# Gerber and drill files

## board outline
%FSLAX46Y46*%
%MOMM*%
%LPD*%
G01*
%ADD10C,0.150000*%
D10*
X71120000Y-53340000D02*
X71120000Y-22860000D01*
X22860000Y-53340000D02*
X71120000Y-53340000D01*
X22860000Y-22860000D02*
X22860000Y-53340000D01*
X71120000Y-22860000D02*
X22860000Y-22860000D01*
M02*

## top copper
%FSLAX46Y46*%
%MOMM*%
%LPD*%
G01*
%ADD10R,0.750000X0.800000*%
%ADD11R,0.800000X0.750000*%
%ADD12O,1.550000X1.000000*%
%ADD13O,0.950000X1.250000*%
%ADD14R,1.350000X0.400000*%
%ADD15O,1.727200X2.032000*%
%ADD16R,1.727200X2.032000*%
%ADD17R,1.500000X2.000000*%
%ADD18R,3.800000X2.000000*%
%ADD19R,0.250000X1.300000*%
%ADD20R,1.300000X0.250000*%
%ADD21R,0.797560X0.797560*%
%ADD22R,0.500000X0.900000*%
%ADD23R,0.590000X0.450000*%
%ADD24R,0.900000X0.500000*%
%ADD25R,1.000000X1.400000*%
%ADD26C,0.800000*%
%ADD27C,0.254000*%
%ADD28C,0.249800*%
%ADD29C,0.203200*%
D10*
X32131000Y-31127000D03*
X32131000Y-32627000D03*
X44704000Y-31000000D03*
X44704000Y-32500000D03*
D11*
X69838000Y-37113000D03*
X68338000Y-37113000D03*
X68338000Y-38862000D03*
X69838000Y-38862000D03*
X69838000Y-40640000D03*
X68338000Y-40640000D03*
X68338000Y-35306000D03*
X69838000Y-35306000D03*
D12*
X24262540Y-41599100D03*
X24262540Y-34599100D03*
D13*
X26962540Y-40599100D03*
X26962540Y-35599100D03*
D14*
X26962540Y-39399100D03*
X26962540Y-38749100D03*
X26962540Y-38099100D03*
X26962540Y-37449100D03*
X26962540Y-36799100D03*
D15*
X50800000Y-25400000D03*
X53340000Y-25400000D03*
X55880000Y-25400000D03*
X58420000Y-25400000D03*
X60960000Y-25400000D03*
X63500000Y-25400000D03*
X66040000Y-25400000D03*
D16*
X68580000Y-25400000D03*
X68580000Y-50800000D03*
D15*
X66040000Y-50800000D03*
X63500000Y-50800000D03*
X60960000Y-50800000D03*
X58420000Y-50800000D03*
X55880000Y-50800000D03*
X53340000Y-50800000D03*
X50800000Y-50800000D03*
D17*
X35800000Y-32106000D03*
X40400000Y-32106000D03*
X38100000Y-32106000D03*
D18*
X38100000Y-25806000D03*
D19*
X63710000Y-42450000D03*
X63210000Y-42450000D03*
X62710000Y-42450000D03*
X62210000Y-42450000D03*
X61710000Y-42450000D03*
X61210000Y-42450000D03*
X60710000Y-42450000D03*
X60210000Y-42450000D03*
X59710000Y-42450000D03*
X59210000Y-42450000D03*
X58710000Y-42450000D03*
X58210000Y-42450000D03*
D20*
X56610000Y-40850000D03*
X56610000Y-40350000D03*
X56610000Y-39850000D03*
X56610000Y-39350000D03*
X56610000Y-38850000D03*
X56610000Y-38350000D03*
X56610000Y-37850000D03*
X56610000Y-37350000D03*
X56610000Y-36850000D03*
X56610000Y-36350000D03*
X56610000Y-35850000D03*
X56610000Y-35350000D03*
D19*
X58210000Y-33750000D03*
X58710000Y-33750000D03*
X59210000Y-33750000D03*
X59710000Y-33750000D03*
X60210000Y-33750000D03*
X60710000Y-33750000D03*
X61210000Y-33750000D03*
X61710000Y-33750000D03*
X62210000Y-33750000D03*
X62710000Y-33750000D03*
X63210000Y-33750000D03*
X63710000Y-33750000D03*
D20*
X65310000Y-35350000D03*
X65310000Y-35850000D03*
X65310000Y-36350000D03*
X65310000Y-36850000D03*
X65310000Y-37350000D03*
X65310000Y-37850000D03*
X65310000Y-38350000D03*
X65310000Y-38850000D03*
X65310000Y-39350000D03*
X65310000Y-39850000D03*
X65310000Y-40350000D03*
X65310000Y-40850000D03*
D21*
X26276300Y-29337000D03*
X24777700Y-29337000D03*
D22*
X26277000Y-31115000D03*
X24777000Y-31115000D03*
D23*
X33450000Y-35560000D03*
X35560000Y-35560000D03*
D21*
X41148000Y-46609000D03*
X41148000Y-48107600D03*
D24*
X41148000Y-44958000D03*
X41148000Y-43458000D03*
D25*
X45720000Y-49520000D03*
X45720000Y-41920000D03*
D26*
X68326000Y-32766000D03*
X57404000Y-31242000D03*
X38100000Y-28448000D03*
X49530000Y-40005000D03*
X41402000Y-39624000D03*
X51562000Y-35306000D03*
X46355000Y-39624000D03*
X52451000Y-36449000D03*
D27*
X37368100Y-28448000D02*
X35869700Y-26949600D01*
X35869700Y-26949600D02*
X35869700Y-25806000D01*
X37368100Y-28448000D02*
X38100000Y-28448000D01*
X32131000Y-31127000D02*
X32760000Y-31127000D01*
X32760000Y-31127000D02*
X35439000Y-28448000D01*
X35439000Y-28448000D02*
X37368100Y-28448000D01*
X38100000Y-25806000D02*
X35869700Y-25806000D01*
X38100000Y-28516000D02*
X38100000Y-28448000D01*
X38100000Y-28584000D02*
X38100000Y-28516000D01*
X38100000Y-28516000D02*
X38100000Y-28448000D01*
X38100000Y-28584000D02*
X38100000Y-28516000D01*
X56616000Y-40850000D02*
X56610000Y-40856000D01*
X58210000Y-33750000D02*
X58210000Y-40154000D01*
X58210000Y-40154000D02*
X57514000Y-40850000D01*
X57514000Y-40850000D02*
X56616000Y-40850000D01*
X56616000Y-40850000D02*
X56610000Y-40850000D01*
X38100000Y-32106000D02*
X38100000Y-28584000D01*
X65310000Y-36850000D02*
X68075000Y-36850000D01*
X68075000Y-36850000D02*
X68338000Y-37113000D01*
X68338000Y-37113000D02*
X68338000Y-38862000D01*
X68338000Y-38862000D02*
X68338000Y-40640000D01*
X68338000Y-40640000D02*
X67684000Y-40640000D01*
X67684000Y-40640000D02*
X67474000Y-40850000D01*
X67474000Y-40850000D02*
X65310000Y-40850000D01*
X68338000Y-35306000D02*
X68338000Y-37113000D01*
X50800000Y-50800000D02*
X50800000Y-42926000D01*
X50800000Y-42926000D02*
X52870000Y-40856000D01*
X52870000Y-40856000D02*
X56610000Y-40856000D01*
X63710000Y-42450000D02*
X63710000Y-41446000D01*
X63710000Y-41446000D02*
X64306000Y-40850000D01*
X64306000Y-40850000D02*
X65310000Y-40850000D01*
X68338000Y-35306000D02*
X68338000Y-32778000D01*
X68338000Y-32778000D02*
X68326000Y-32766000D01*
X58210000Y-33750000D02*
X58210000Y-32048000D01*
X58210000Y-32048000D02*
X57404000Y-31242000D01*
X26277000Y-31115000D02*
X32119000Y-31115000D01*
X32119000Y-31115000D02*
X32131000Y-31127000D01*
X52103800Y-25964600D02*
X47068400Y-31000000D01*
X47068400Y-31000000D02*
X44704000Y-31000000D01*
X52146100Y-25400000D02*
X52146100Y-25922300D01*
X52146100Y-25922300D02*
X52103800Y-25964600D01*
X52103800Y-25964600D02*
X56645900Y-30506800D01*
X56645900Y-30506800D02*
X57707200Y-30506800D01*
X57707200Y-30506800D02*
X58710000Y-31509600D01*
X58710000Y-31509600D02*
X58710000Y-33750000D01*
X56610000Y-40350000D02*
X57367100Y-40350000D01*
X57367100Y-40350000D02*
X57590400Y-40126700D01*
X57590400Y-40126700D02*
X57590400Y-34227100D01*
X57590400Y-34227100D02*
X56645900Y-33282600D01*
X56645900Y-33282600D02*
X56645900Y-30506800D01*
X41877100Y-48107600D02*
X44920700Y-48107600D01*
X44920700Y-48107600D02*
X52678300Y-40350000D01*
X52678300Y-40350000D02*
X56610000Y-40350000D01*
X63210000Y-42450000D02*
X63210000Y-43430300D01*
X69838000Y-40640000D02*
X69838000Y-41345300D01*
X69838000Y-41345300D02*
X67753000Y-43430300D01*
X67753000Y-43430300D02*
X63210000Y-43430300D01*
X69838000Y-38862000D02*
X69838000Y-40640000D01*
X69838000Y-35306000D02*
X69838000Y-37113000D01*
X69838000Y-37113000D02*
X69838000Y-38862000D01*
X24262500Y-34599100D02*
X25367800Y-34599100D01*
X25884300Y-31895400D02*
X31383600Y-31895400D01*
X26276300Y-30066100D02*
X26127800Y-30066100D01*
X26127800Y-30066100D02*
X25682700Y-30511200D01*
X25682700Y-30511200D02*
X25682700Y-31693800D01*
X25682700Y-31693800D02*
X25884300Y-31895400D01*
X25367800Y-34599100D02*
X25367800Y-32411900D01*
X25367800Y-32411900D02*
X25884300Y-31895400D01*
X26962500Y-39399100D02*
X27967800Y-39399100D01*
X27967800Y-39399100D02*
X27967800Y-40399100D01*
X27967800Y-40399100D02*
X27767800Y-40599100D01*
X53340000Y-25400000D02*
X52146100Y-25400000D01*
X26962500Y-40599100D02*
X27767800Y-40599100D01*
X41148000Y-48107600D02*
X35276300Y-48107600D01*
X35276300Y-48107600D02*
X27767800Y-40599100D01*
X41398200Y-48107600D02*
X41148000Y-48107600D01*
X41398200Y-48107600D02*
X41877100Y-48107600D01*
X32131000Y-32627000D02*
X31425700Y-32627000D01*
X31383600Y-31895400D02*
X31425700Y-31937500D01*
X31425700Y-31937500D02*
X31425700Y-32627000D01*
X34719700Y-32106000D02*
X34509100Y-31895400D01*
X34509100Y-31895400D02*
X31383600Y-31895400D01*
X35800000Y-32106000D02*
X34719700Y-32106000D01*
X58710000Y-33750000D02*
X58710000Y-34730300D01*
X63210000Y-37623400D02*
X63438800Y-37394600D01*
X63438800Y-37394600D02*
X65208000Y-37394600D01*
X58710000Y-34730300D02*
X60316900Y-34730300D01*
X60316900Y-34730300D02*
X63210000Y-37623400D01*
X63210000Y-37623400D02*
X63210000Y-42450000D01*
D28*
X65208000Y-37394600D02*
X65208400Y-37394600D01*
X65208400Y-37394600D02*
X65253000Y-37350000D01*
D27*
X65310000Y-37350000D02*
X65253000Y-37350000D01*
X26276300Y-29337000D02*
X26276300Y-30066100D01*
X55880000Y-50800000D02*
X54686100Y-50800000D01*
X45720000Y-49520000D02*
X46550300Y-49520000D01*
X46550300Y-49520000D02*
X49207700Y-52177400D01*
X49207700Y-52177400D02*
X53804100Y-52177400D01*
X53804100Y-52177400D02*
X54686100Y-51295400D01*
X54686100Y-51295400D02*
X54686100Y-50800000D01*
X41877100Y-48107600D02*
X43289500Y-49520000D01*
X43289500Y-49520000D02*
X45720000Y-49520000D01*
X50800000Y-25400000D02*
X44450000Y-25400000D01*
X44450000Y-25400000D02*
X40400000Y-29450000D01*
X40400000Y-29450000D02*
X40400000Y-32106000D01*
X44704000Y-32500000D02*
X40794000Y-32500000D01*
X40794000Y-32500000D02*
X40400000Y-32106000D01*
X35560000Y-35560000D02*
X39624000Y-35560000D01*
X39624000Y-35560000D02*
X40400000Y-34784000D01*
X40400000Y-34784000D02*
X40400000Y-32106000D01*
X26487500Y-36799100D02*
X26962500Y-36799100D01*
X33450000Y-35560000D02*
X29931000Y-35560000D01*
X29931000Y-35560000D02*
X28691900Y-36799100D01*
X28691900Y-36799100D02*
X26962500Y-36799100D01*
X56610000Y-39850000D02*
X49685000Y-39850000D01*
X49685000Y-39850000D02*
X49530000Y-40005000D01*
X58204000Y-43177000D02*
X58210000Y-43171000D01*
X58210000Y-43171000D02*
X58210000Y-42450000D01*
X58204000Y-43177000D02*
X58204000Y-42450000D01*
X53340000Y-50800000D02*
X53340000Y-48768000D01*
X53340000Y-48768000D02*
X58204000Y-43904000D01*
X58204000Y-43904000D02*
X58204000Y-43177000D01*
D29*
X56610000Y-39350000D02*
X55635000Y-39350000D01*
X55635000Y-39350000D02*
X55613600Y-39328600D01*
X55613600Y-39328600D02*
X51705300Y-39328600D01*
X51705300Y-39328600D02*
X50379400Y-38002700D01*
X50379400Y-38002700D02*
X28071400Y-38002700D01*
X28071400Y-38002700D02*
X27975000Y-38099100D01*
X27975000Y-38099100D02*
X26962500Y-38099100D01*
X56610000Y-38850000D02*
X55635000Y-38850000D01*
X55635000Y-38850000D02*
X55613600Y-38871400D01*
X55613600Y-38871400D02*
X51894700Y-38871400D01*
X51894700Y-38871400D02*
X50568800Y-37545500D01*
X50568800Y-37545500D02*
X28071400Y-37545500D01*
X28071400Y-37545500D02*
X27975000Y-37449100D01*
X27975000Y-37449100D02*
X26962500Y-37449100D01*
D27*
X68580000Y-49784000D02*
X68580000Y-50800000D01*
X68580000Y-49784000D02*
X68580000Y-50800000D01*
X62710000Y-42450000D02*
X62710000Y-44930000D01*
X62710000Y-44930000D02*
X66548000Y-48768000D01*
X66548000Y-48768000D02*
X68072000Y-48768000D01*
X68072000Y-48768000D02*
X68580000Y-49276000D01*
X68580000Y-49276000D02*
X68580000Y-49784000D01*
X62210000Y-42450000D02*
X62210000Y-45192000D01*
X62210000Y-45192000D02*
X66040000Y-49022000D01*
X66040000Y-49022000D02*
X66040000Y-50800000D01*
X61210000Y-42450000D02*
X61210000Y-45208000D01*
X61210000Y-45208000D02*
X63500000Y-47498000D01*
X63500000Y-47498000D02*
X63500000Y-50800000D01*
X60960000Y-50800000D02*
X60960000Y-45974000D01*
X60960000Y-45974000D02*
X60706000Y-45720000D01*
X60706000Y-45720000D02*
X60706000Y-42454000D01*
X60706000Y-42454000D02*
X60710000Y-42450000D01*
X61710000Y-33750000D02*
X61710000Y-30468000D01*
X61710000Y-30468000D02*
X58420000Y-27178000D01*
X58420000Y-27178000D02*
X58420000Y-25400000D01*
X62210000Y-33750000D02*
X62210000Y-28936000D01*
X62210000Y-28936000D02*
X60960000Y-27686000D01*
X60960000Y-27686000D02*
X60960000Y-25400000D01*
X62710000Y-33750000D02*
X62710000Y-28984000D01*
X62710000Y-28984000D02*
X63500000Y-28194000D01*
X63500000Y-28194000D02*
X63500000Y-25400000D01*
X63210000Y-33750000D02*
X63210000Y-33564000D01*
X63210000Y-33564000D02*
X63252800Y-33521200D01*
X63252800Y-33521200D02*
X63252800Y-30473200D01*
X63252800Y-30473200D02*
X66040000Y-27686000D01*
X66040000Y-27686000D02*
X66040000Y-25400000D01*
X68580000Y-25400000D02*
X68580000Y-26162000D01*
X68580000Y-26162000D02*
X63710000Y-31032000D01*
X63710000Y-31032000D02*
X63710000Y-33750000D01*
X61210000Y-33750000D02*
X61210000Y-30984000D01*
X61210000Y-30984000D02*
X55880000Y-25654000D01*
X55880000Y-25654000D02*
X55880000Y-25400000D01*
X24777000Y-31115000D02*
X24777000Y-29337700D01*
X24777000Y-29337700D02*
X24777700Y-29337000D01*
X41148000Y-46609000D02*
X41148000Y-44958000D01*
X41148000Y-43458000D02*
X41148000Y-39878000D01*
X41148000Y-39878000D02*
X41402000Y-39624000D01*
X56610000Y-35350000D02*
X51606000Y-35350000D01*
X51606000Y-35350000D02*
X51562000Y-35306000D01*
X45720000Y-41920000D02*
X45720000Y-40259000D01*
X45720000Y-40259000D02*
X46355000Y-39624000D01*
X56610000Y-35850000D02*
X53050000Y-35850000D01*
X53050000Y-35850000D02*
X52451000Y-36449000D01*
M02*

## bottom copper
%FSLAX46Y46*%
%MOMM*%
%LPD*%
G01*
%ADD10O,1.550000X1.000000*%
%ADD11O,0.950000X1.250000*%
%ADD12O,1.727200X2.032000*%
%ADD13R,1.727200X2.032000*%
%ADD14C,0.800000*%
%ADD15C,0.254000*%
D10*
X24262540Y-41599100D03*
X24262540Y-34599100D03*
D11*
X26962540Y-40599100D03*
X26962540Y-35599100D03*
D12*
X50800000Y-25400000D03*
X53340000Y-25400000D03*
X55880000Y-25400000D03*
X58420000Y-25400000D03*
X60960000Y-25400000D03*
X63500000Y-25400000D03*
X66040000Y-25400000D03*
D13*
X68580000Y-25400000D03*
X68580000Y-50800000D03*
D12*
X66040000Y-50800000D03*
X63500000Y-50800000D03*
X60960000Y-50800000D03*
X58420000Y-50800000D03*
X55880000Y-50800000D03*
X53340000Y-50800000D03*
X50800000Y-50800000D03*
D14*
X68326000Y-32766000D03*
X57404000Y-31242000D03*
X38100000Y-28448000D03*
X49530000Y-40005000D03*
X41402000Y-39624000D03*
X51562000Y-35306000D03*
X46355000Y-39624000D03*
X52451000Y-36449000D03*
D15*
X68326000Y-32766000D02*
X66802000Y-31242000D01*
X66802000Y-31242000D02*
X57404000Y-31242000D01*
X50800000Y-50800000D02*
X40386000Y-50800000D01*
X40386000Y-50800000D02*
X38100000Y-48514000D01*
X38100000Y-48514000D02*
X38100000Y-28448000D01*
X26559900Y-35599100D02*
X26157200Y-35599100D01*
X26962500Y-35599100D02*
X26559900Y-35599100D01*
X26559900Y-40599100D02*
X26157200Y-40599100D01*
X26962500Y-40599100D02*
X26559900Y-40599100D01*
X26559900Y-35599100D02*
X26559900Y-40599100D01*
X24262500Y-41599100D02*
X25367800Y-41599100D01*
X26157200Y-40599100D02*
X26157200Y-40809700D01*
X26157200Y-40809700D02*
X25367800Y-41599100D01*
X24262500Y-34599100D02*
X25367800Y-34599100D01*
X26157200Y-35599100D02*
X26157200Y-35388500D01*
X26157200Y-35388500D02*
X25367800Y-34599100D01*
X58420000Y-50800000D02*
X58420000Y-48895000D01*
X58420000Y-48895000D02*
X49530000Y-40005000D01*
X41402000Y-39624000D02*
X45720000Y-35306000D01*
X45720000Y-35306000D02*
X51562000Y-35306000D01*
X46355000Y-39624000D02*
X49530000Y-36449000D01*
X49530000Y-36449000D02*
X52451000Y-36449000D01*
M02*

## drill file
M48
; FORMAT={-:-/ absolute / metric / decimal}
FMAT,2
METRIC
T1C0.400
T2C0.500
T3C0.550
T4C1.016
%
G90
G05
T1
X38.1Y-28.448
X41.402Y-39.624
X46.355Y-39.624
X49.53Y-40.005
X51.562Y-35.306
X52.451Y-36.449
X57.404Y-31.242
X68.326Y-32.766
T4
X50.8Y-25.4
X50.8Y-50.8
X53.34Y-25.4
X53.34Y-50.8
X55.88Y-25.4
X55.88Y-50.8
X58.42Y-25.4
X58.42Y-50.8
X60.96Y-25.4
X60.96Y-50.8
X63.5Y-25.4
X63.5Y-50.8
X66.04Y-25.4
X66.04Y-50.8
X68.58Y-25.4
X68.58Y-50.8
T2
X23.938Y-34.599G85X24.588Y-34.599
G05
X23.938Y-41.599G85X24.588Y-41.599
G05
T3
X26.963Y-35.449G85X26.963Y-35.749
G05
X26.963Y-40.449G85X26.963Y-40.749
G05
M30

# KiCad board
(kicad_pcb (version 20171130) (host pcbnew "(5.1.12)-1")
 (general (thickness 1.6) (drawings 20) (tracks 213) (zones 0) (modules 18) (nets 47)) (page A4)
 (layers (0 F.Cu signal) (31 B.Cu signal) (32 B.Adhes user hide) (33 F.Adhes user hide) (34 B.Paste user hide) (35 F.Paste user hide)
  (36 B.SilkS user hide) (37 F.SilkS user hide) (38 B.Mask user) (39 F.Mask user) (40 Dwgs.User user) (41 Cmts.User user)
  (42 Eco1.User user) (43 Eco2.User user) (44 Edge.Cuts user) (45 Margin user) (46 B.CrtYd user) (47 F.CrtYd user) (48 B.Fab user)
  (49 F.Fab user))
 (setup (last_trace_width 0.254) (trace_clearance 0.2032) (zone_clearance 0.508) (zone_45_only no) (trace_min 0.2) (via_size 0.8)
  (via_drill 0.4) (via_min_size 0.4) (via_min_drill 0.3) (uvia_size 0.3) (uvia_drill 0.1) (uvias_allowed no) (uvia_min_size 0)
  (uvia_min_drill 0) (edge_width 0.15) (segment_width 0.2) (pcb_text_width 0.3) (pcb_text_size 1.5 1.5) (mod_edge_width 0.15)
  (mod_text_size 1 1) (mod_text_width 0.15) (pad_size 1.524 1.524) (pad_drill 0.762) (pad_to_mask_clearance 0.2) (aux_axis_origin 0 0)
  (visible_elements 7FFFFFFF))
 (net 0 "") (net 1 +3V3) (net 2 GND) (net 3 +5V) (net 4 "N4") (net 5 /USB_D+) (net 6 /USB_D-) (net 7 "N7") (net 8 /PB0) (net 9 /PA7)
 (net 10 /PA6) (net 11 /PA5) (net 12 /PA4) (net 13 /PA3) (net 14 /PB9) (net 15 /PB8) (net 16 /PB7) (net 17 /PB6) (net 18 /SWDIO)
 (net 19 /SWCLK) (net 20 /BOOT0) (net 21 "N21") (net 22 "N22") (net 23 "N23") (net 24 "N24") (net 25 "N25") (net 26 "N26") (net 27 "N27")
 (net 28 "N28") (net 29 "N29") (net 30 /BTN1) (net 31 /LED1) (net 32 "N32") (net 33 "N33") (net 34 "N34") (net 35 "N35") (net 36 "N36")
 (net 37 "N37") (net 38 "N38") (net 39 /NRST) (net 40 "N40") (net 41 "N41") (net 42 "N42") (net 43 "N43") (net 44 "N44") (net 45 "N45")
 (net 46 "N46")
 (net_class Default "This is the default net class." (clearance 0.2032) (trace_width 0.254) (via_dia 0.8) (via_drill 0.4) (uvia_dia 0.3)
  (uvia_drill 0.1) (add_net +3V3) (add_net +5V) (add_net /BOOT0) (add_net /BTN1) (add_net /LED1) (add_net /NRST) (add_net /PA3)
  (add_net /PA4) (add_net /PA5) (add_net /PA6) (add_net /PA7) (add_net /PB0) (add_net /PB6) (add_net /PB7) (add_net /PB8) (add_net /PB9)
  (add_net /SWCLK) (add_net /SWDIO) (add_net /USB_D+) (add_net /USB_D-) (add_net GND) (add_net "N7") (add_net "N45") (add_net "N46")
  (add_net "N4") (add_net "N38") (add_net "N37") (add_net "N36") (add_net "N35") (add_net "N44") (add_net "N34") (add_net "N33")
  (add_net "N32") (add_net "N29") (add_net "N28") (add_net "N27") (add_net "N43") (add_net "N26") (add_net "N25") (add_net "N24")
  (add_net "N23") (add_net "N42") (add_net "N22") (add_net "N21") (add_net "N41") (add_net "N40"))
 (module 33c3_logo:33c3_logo (layer F.Cu) (at 31.75 46.101)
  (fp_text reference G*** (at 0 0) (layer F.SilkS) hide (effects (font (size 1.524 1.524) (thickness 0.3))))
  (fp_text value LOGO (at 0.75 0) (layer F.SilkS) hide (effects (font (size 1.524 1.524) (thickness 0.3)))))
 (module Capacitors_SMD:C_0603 (layer F.Cu) (at 32.131 31.877 270)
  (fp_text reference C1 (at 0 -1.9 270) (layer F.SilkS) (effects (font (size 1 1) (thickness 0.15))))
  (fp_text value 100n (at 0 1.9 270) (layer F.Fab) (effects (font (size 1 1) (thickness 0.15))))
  (pad 1 smd rect (at -0.75 0 270) (size 0.8 0.75) (layers F.Cu F.Paste F.Mask) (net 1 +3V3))
  (pad 2 smd rect (at 0.75 0 270) (size 0.8 0.75) (layers F.Cu F.Paste F.Mask) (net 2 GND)))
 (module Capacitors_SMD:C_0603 (layer F.Cu) (at 44.704 31.75 90)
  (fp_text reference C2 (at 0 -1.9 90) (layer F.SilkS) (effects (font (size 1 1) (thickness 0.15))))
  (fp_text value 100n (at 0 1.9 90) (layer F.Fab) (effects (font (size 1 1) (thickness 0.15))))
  (pad 2 smd rect (at 0.75 0 90) (size 0.8 0.75) (layers F.Cu F.Paste F.Mask) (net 2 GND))
  (pad 1 smd rect (at -0.75 0 90) (size 0.8 0.75) (layers F.Cu F.Paste F.Mask) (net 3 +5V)))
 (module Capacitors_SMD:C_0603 (layer F.Cu) (at 69.088 37.113)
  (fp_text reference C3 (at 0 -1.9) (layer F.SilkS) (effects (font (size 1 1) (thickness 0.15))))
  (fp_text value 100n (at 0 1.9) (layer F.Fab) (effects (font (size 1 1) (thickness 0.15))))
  (pad 2 smd rect (at 0.75 0) (size 0.8 0.75) (layers F.Cu F.Paste F.Mask) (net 2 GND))
  (pad 1 smd rect (at -0.75 0) (size 0.8 0.75) (layers F.Cu F.Paste F.Mask) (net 1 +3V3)))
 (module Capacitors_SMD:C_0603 (layer F.Cu) (at 69.088 38.862)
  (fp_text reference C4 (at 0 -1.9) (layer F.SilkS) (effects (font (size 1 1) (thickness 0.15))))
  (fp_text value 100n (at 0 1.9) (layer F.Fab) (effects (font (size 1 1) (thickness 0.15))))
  (pad 1 smd rect (at -0.75 0) (size 0.8 0.75) (layers F.Cu F.Paste F.Mask) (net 1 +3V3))
  (pad 2 smd rect (at 0.75 0) (size 0.8 0.75) (layers F.Cu F.Paste F.Mask) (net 2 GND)))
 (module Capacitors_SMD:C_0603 (layer F.Cu) (at 69.088 40.64)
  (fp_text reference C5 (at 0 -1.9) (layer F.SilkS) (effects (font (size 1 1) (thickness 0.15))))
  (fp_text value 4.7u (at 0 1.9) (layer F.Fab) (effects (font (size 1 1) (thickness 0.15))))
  (pad 2 smd rect (at 0.75 0) (size 0.8 0.75) (layers F.Cu F.Paste F.Mask) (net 2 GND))
  (pad 1 smd rect (at -0.75 0) (size 0.8 0.75) (layers F.Cu F.Paste F.Mask) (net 1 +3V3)))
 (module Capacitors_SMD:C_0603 (layer F.Cu) (at 69.088 35.306)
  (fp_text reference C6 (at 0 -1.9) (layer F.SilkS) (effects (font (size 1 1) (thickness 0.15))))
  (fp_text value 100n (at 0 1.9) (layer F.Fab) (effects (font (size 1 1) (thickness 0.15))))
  (pad 1 smd rect (at -0.75 0) (size 0.8 0.75) (layers F.Cu F.Paste F.Mask) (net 1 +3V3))
  (pad 2 smd rect (at 0.75 0) (size 0.8 0.75) (layers F.Cu F.Paste F.Mask) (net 2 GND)))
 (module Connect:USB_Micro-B (layer F.Cu) (at 25.4 38.1 270)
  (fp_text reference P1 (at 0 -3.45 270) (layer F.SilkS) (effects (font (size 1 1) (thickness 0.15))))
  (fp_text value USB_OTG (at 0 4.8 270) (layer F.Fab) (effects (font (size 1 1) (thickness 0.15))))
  (pad 6 thru_hole oval (at 3.4991 1.13746) (size 1.55 1) (drill oval 1.15 0.5) (layers *.Cu *.Mask) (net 2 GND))
  (pad 6 thru_hole oval (at -3.5009 1.13746) (size 1.55 1) (drill oval 1.15 0.5) (layers *.Cu *.Mask) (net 2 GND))
  (pad 6 thru_hole oval (at 2.4991 -1.56254) (size 0.95 1.25) (drill oval 0.55 0.85) (layers *.Cu *.Mask) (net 2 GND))
  (pad 6 thru_hole oval (at -2.5009 -1.56254) (size 0.95 1.25) (drill oval 0.55 0.85) (layers *.Cu *.Mask) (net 2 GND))
  (pad 5 smd rect (at 1.2991 -1.56254) (size 1.35 0.4) (layers F.Cu F.Paste F.Mask) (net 2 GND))
  (pad 4 smd rect (at 0.6491 -1.56254) (size 1.35 0.4) (layers F.Cu F.Paste F.Mask) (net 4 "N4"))
  (pad 3 smd rect (at -0.0009 -1.56254) (size 1.35 0.4) (layers F.Cu F.Paste F.Mask) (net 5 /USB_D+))
  (pad 2 smd rect (at -0.6509 -1.56254) (size 1.35 0.4) (layers F.Cu F.Paste F.Mask) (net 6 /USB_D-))
  (pad 1 smd rect (at -1.3009 -1.56254) (size 1.35 0.4) (layers F.Cu F.Paste F.Mask) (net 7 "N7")))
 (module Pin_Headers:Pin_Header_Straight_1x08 (layer F.Cu) (at 68.58 25.4 270)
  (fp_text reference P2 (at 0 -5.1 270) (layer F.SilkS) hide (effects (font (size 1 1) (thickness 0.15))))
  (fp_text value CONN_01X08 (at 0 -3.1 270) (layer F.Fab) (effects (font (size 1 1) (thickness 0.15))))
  (pad 8 thru_hole oval (at 0 17.78 270) (size 2.032 1.7272) (drill 1.016) (layers *.Cu *.Mask) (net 3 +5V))
  (pad 7 thru_hole oval (at 0 15.24 270) (size 2.032 1.7272) (drill 1.016) (layers *.Cu *.Mask) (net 2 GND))
  (pad 6 thru_hole oval (at 0 12.7 270) (size 2.032 1.7272) (drill 1.016) (layers *.Cu *.Mask) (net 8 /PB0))
  (pad 5 thru_hole oval (at 0 10.16 270) (size 2.032 1.7272) (drill 1.016) (layers *.Cu *.Mask) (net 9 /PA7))
  (pad 4 thru_hole oval (at 0 7.62 270) (size 2.032 1.7272) (drill 1.016) (layers *.Cu *.Mask) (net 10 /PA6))
  (pad 3 thru_hole oval (at 0 5.08 270) (size 2.032 1.7272) (drill 1.016) (layers *.Cu *.Mask) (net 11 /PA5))
  (pad 2 thru_hole oval (at 0 2.54 270) (size 2.032 1.7272) (drill 1.016) (layers *.Cu *.Mask) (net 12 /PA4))
  (pad 1 thru_hole rect (at 0 0 270) (size 2.032 1.7272) (drill 1.016) (layers *.Cu *.Mask) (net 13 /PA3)))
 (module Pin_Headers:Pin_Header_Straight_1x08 (layer F.Cu) (at 68.58 50.8 270)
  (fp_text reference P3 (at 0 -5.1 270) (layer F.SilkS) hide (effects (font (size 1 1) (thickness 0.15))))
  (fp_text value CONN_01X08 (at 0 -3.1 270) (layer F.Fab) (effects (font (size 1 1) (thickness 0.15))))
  (pad 1 thru_hole rect (at 0 0 270) (size 2.032 1.7272) (drill 1.016) (layers *.Cu *.Mask) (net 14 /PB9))
  (pad 2 thru_hole oval (at 0 2.54 270) (size 2.032 1.7272) (drill 1.016) (layers *.Cu *.Mask) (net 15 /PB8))
  (pad 3 thru_hole oval (at 0 5.08 270) (size 2.032 1.7272) (drill 1.016) (layers *.Cu *.Mask) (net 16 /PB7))
  (pad 4 thru_hole oval (at 0 7.62 270) (size 2.032 1.7272) (drill 1.016) (layers *.Cu *.Mask) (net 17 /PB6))
  (pad 5 thru_hole oval (at 0 10.16 270) (size 2.032 1.7272) (drill 1.016) (layers *.Cu *.Mask) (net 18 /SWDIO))
  (pad 6 thru_hole oval (at 0 12.7 270) (size 2.032 1.7272) (drill 1.016) (layers *.Cu *.Mask) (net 2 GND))
  (pad 7 thru_hole oval (at 0 15.24 270) (size 2.032 1.7272) (drill 1.016) (layers *.Cu *.Mask) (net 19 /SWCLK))
  (pad 8 thru_hole oval (at 0 17.78 270) (size 2.032 1.7272) (drill 1.016) (layers *.Cu *.Mask) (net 1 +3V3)))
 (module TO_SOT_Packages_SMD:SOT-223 (layer F.Cu) (at 38.1 28.956 90)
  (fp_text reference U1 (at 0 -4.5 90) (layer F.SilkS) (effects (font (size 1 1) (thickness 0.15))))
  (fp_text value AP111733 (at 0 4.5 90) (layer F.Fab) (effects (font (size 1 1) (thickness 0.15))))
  (pad 1 smd rect (at -3.15 -2.3 90) (size 2 1.5) (layers F.Cu F.Paste F.Mask) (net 2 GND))
  (pad 3 smd rect (at -3.15 2.3 90) (size 2 1.5) (layers F.Cu F.Paste F.Mask) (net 3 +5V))
  (pad 2 smd rect (at -3.15 0 90) (size 2 1.5) (layers F.Cu F.Paste F.Mask) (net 1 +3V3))
  (pad 4 smd rect (at 3.15 0 90) (size 2 3.8) (layers F.Cu F.Paste F.Mask) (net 1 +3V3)))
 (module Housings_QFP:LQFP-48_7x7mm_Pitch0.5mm (layer F.Cu) (at 60.96 38.1 180)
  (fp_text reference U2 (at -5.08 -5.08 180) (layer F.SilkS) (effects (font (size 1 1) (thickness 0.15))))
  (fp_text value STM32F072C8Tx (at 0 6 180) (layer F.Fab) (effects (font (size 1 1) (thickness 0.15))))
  (pad 48 smd rect (at -2.75 -4.35 270) (size 1.3 0.25) (layers F.Cu F.Paste F.Mask) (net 1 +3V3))
  (pad 47 smd rect (at -2.25 -4.35 270) (size 1.3 0.25) (layers F.Cu F.Paste F.Mask) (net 2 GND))
  (pad 46 smd rect (at -1.75 -4.35 270) (size 1.3 0.25) (layers F.Cu F.Paste F.Mask) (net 14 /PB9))
  (pad 45 smd rect (at -1.25 -4.35 270) (size 1.3 0.25) (layers F.Cu F.Paste F.Mask) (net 15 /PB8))
  (pad 44 smd rect (at -0.75 -4.35 270) (size 1.3 0.25) (layers F.Cu F.Paste F.Mask) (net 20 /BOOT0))
  (pad 43 smd rect (at -0.25 -4.35 270) (size 1.3 0.25) (layers F.Cu F.Paste F.Mask) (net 16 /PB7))
  (pad 42 smd rect (at 0.25 -4.35 270) (size 1.3 0.25) (layers F.Cu F.Paste F.Mask) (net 17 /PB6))
  (pad 41 smd rect (at 0.75 -4.35 270) (size 1.3 0.25) (layers F.Cu F.Paste F.Mask) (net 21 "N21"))
  (pad 40 smd rect (at 1.25 -4.35 270) (size 1.3 0.25) (layers F.Cu F.Paste F.Mask) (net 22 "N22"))
  (pad 39 smd rect (at 1.75 -4.35 270) (size 1.3 0.25) (layers F.Cu F.Paste F.Mask) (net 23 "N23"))
  (pad 38 smd rect (at 2.25 -4.35 270) (size 1.3 0.25) (layers F.Cu F.Paste F.Mask) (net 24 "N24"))
  (pad 37 smd rect (at 2.75 -4.35 270) (size 1.3 0.25) (layers F.Cu F.Paste F.Mask) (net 19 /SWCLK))
  (pad 36 smd rect (at 4.35 -2.75 180) (size 1.3 0.25) (layers F.Cu F.Paste F.Mask) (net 1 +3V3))
  (pad 35 smd rect (at 4.35 -2.25 180) (size 1.3 0.25) (layers F.Cu F.Paste F.Mask) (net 2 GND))
  (pad 34 smd rect (at 4.35 -1.75 180) (size 1.3 0.25) (layers F.Cu F.Paste F.Mask) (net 18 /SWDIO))
  (pad 33 smd rect (at 4.35 -1.25 180) (size 1.3 0.25) (layers F.Cu F.Paste F.Mask) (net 5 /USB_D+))
  (pad 32 smd rect (at 4.35 -0.75 180) (size 1.3 0.25) (layers F.Cu F.Paste F.Mask) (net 6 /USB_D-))
  (pad 31 smd rect (at 4.35 -0.25 180) (size 1.3 0.25) (layers F.Cu F.Paste F.Mask) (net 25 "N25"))
  (pad 30 smd rect (at 4.35 0.25 180) (size 1.3 0.25) (layers F.Cu F.Paste F.Mask) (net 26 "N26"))
  (pad 29 smd rect (at 4.35 0.75 180) (size 1.3 0.25) (layers F.Cu F.Paste F.Mask) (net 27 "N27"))
  (pad 28 smd rect (at 4.35 1.25 180) (size 1.3 0.25) (layers F.Cu F.Paste F.Mask) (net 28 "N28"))
  (pad 27 smd rect (at 4.35 1.75 180) (size 1.3 0.25) (layers F.Cu F.Paste F.Mask) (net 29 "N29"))
  (pad 26 smd rect (at 4.35 2.25 180) (size 1.3 0.25) (layers F.Cu F.Paste F.Mask) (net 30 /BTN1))
  (pad 25 smd rect (at 4.35 2.75 180) (size 1.3 0.25) (layers F.Cu F.Paste F.Mask) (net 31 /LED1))
  (pad 24 smd rect (at 2.75 4.35 270) (size 1.3 0.25) (layers F.Cu F.Paste F.Mask) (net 1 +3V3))
  (pad 23 smd rect (at 2.25 4.35 270) (size 1.3 0.25) (layers F.Cu F.Paste F.Mask) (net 2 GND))
  (pad 22 smd rect (at 1.75 4.35 270) (size 1.3 0.25) (layers F.Cu F.Paste F.Mask) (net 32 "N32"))
  (pad 21 smd rect (at 1.25 4.35 270) (size 1.3 0.25) (layers F.Cu F.Paste F.Mask) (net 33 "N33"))
  (pad 20 smd rect (at 0.75 4.35 270) (size 1.3 0.25) (layers F.Cu F.Paste F.Mask) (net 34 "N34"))
  (pad 19 smd rect (at 0.25 4.35 270) (size 1.3 0.25) (layers F.Cu F.Paste F.Mask) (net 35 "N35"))
  (pad 18 smd rect (at -0.25 4.35 270) (size 1.3 0.25) (layers F.Cu F.Paste F.Mask) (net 8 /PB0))
  (pad 17 smd rect (at -0.75 4.35 270) (size 1.3 0.25) (layers F.Cu F.Paste F.Mask) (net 9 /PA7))
  (pad 16 smd rect (at -1.25 4.35 270) (size 1.3 0.25) (layers F.Cu F.Paste F.Mask) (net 10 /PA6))
  (pad 15 smd rect (at -1.75 4.35 270) (size 1.3 0.25) (layers F.Cu F.Paste F.Mask) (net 11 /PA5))
  (pad 14 smd rect (at -2.25 4.35 270) (size 1.3 0.25) (layers F.Cu F.Paste F.Mask) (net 12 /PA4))
  (pad 13 smd rect (at -2.75 4.35 270) (size 1.3 0.25) (layers F.Cu F.Paste F.Mask) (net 13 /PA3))
  (pad 12 smd rect (at -4.35 2.75 180) (size 1.3 0.25) (layers F.Cu F.Paste F.Mask) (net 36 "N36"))
  (pad 11 smd rect (at -4.35 2.25 180) (size 1.3 0.25) (layers F.Cu F.Paste F.Mask) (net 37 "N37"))
  (pad 10 smd rect (at -4.35 1.75 180) (size 1.3 0.25) (layers F.Cu F.Paste F.Mask) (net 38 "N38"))
  (pad 9 smd rect (at -4.35 1.25 180) (size 1.3 0.25) (layers F.Cu F.Paste F.Mask) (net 1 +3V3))
  (pad 8 smd rect (at -4.35 0.75 180) (size 1.3 0.25) (layers F.Cu F.Paste F.Mask) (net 2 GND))
  (pad 7 smd rect (at -4.35 0.25 180) (size 1.3 0.25) (layers F.Cu F.Paste F.Mask) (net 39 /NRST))
  (pad 6 smd rect (at -4.35 -0.25 180) (size 1.3 0.25) (layers F.Cu F.Paste F.Mask) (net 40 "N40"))
  (pad 5 smd rect (at -4.35 -0.75 180) (size 1.3 0.25) (layers F.Cu F.Paste F.Mask) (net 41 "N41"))
  (pad 4 smd rect (at -4.35 -1.25 180) (size 1.3 0.25) (layers F.Cu F.Paste F.Mask) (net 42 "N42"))
  (pad 3 smd rect (at -4.35 -1.75 180) (size 1.3 0.25) (layers F.Cu F.Paste F.Mask) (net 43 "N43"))
  (pad 2 smd rect (at -4.35 -2.25 180) (size 1.3 0.25) (layers F.Cu F.Paste F.Mask) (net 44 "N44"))
  (pad 1 smd rect (at -4.35 -2.75 180) (size 1.3 0.25) (layers F.Cu F.Paste F.Mask) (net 1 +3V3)))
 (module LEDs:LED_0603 (layer F.Cu) (at 25.527 29.337 180)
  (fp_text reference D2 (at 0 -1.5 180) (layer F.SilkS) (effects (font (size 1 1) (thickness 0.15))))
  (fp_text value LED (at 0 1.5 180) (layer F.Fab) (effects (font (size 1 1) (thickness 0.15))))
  (pad 1 smd rect (at -0.7493 0) (size 0.79756 0.79756) (layers F.Cu F.Paste F.Mask) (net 2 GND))
  (pad 2 smd rect (at 0.7493 0) (size 0.79756 0.79756) (layers F.Cu F.Paste F.Mask) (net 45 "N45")))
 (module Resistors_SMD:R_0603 (layer F.Cu) (at 25.527 31.115)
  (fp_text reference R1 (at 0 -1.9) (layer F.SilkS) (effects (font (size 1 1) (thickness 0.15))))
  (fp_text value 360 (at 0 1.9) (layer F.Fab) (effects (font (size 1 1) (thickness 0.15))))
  (pad 2 smd rect (at 0.75 0) (size 0.5 0.9) (layers F.Cu F.Paste F.Mask) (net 1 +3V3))
  (pad 1 smd rect (at -0.75 0) (size 0.5 0.9) (layers F.Cu F.Paste F.Mask) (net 45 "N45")))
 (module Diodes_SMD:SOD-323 (layer F.Cu) (at 34.505 35.56 180)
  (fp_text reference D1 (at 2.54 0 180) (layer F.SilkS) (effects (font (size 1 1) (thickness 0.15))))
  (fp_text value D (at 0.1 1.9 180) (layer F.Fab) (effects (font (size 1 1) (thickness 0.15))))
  (pad 2 smd rect (at 1.055 0 180) (size 0.59 0.45) (layers F.Cu F.Paste F.Mask) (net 7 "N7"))
  (pad 1 smd rect (at -1.055 0 180) (size 0.59 0.45) (layers F.Cu F.Paste F.Mask) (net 3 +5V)))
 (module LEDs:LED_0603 (layer F.Cu) (at 41.148 47.3583 90)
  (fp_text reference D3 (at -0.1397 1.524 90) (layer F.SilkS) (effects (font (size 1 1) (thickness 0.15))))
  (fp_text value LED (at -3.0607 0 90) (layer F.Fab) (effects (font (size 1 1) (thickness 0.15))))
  (pad 2 smd rect (at 0.7493 0 270) (size 0.79756 0.79756) (layers F.Cu F.Paste F.Mask) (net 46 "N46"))
  (pad 1 smd rect (at -0.7493 0 270) (size 0.79756 0.79756) (layers F.Cu F.Paste F.Mask) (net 2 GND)))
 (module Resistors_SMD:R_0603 (layer F.Cu) (at 41.148 44.208 90)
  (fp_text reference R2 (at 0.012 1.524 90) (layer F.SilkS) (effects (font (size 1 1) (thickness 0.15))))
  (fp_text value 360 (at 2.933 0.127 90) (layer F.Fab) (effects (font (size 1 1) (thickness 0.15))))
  (pad 1 smd rect (at -0.75 0 90) (size 0.5 0.9) (layers F.Cu F.Paste F.Mask) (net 46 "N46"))
  (pad 2 smd rect (at 0.75 0 90) (size 0.5 0.9) (layers F.Cu F.Paste F.Mask) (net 31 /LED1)))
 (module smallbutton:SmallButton (layer F.Cu) (at 45.72 45.72)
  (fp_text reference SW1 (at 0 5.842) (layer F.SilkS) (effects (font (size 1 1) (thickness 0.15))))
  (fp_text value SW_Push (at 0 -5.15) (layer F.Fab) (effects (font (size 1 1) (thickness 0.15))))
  (pad 2 smd rect (at 0 3.8) (size 1 1.4) (layers F.Cu F.Paste F.Mask) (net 2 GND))
  (pad 1 smd rect (at 0 -3.8) (size 1 1.4) (layers F.Cu F.Paste F.Mask) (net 30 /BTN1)))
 (gr_line (start 71.12 53.34) (end 71.12 22.86) (layer Edge.Cuts) (width 0.15))
 (gr_line (start 22.86 53.34) (end 71.12 53.34) (layer Edge.Cuts) (width 0.15))
 (gr_line (start 22.86 22.86) (end 22.86 53.34) (layer Edge.Cuts) (width 0.15))
 (gr_line (start 71.12 22.86) (end 22.86 22.86) (layer Edge.Cuts) (width 0.15))
 (segment (start 37.3681 28.448) (end 35.8697 26.9496) (width 0.254) (layer F.Cu) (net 1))
 (segment (start 35.8697 26.9496) (end 35.8697 25.806) (width 0.254) (layer F.Cu) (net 1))
 (segment (start 37.3681 28.448) (end 38.1 28.448) (width 0.254) (layer F.Cu) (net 1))
 (segment (start 32.131 31.127) (end 32.76 31.127) (width 0.254) (layer F.Cu) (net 1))
 (segment (start 32.76 31.127) (end 35.439 28.448) (width 0.254) (layer F.Cu) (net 1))
 (segment (start 35.439 28.448) (end 37.3681 28.448) (width 0.254) (layer F.Cu) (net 1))
 (segment (start 38.1 25.806) (end 35.8697 25.806) (width 0.254) (layer F.Cu) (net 1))
 (segment (start 38.1 28.516) (end 38.1 28.448) (width 0.254) (layer F.Cu) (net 1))
 (segment (start 38.1 28.584) (end 38.1 28.516) (width 0.254) (layer F.Cu) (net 1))
 (segment (start 38.1 28.516) (end 38.1 28.448) (width 0.254) (layer F.Cu) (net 1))
 (segment (start 38.1 28.584) (end 38.1 28.516) (width 0.254) (layer F.Cu) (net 1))
 (segment (start 56.616 40.85) (end 56.61 40.856) (width 0.254) (layer F.Cu) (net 1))
 (segment (start 58.21 33.75) (end 58.21 40.154) (width 0.254) (layer F.Cu) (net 1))
 (segment (start 58.21 40.154) (end 57.514 40.85) (width 0.254) (layer F.Cu) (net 1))
 (segment (start 57.514 40.85) (end 56.616 40.85) (width 0.254) (layer F.Cu) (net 1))
 (segment (start 56.616 40.85) (end 56.61 40.85) (width 0.254) (layer F.Cu) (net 1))
 (segment (start 38.1 32.106) (end 38.1 28.584) (width 0.254) (layer F.Cu) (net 1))
 (segment (start 65.31 36.85) (end 68.075 36.85) (width 0.254) (layer F.Cu) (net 1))
 (segment (start 68.075 36.85) (end 68.338 37.113) (width 0.254) (layer F.Cu) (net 1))
 (segment (start 68.338 37.113) (end 68.338 38.862) (width 0.254) (layer F.Cu) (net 1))
 (segment (start 68.338 38.862) (end 68.338 40.64) (width 0.254) (layer F.Cu) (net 1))
 (segment (start 68.338 40.64) (end 67.684 40.64) (width 0.254) (layer F.Cu) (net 1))
 (segment (start 67.684 40.64) (end 67.474 40.85) (width 0.254) (layer F.Cu) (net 1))
 (segment (start 67.474 40.85) (end 65.31 40.85) (width 0.254) (layer F.Cu) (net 1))
 (segment (start 68.338 35.306) (end 68.338 37.113) (width 0.254) (layer F.Cu) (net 1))
 (segment (start 50.8 50.8) (end 50.8 42.926) (width 0.254) (layer F.Cu) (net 1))
 (segment (start 50.8 42.926) (end 52.87 40.856) (width 0.254) (layer F.Cu) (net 1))
 (segment (start 52.87 40.856) (end 56.61 40.856) (width 0.254) (layer F.Cu) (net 1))
 (segment (start 63.71 42.45) (end 63.71 41.446) (width 0.254) (layer F.Cu) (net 1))
 (segment (start 63.71 41.446) (end 64.306 40.85) (width 0.254) (layer F.Cu) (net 1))
 (segment (start 64.306 40.85) (end 65.31 40.85) (width 0.254) (layer F.Cu) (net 1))
 (segment (start 68.338 35.306) (end 68.338 32.778) (width 0.254) (layer F.Cu) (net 1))
 (segment (start 68.338 32.778) (end 68.326 32.766) (width 0.254) (layer F.Cu) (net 1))
 (segment (start 68.326 32.766) (end 66.802 31.242) (width 0.254) (layer B.Cu) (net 1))
 (segment (start 66.802 31.242) (end 57.404 31.242) (width 0.254) (layer B.Cu) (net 1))
 (segment (start 58.21 33.75) (end 58.21 32.048) (width 0.254) (layer F.Cu) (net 1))
 (segment (start 58.21 32.048) (end 57.404 31.242) (width 0.254) (layer F.Cu) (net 1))
 (segment (start 50.8 50.8) (end 40.386 50.8) (width 0.254) (layer B.Cu) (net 1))
 (segment (start 40.386 50.8) (end 38.1 48.514) (width 0.254) (layer B.Cu) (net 1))
 (segment (start 38.1 48.514) (end 38.1 28.448) (width 0.254) (layer B.Cu) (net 1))
 (segment (start 26.277 31.115) (end 32.119 31.115) (width 0.254) (layer F.Cu) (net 1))
 (segment (start 32.119 31.115) (end 32.131 31.127) (width 0.254) (layer F.Cu) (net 1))
 (via (at 68.326 32.766) (size 0.8) (layers F.Cu B.Cu) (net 1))
 (via (at 57.404 31.242) (size 0.8) (layers F.Cu B.Cu) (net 1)) (via (at 38.1 28.448) (size 0.8) (layers F.Cu B.Cu) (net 1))
 (segment (start 52.1038 25.9646) (end 47.0684 31) (width 0.254) (layer F.Cu) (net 2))
 (segment (start 47.0684 31) (end 44.704 31) (width 0.254) (layer F.Cu) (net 2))
 (segment (start 52.1461 25.4) (end 52.1461 25.9223) (width 0.254) (layer F.Cu) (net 2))
 (segment (start 52.1461 25.9223) (end 52.1038 25.9646) (width 0.254) (layer F.Cu) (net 2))
 (segment (start 52.1038 25.9646) (end 56.6459 30.5068) (width 0.254) (layer F.Cu) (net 2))
 (segment (start 56.6459 30.5068) (end 57.7072 30.5068) (width 0.254) (layer F.Cu) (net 2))
 (segment (start 57.7072 30.5068) (end 58.71 31.5096) (width 0.254) (layer F.Cu) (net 2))
 (segment (start 58.71 31.5096) (end 58.71 33.75) (width 0.254) (layer F.Cu) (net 2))
 (segment (start 56.61 40.35) (end 57.3671 40.35) (width 0.254) (layer F.Cu) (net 2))
 (segment (start 57.3671 40.35) (end 57.5904 40.1267) (width 0.254) (layer F.Cu) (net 2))
 (segment (start 57.5904 40.1267) (end 57.5904 34.2271) (width 0.254) (layer F.Cu) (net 2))
 (segment (start 57.5904 34.2271) (end 56.6459 33.2826) (width 0.254) (layer F.Cu) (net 2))
 (segment (start 56.6459 33.2826) (end 56.6459 30.5068) (width 0.254) (layer F.Cu) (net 2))
 (segment (start 41.8771 48.1076) (end 44.9207 48.1076) (width 0.254) (layer F.Cu) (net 2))
 (segment (start 44.9207 48.1076) (end 52.6783 40.35) (width 0.254) (layer F.Cu) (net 2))
 (segment (start 52.6783 40.35) (end 56.61 40.35) (width 0.254) (layer F.Cu) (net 2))
 (segment (start 63.21 42.45) (end 63.21 43.4303) (width 0.254) (layer F.Cu) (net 2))
 (segment (start 69.838 40.64) (end 69.838 41.3453) (width 0.254) (layer F.Cu) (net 2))
 (segment (start 69.838 41.3453) (end 67.753 43.4303) (width 0.254) (layer F.Cu) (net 2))
 (segment (start 67.753 43.4303) (end 63.21 43.4303) (width 0.254) (layer F.Cu) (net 2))
 (segment (start 69.838 38.862) (end 69.838 40.64) (width 0.254) (layer F.Cu) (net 2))
 (segment (start 69.838 35.306) (end 69.838 37.113) (width 0.254) (layer F.Cu) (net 2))
 (segment (start 69.838 37.113) (end 69.838 38.862) (width 0.254) (layer F.Cu) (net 2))
 (segment (start 24.2625 34.5991) (end 25.3678 34.5991) (width 0.254) (layer F.Cu) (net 2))
 (segment (start 25.8843 31.8954) (end 31.3836 31.8954) (width 0.254) (layer F.Cu) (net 2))
 (segment (start 26.2763 30.0661) (end 26.1278 30.0661) (width 0.254) (layer F.Cu) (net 2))
 (segment (start 26.1278 30.0661) (end 25.6827 30.5112) (width 0.254) (layer F.Cu) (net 2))
 (segment (start 25.6827 30.5112) (end 25.6827 31.6938) (width 0.254) (layer F.Cu) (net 2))
 (segment (start 25.6827 31.6938) (end 25.8843 31.8954) (width 0.254) (layer F.Cu) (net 2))
 (segment (start 25.3678 34.5991) (end 25.3678 32.4119) (width 0.254) (layer F.Cu) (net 2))
 (segment (start 25.3678 32.4119) (end 25.8843 31.8954) (width 0.254) (layer F.Cu) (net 2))
 (segment (start 26.5599 35.5991) (end 26.1572 35.5991) (width 0.254) (layer B.Cu) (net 2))
 (segment (start 26.9625 35.5991) (end 26.5599 35.5991) (width 0.254) (layer B.Cu) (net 2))
 (segment (start 26.5599 40.5991) (end 26.1572 40.5991) (width 0.254) (layer B.Cu) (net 2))
 (segment (start 26.9625 40.5991) (end 26.5599 40.5991) (width 0.254) (layer B.Cu) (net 2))
 (segment (start 26.5599 35.5991) (end 26.5599 40.5991) (width 0.254) (layer B.Cu) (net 2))
 (segment (start 24.2625 41.5991) (end 25.3678 41.5991) (width 0.254) (layer B.Cu) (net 2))
 (segment (start 26.1572 40.5991) (end 26.1572 40.8097) (width 0.254) (layer B.Cu) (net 2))
 (segment (start 26.1572 40.8097) (end 25.3678 41.5991) (width 0.254) (layer B.Cu) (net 2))
 (segment (start 24.2625 34.5991) (end 25.3678 34.5991) (width 0.254) (layer B.Cu) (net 2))
 (segment (start 26.1572 35.5991) (end 26.1572 35.3885) (width 0.254) (layer B.Cu) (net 2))
 (segment (start 26.1572 35.3885) (end 25.3678 34.5991) (width 0.254) (layer B.Cu) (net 2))
 (segment (start 26.9625 39.3991) (end 27.9678 39.3991) (width 0.254) (layer F.Cu) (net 2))
 (segment (start 27.9678 39.3991) (end 27.9678 40.3991) (width 0.254) (layer F.Cu) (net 2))
 (segment (start 27.9678 40.3991) (end 27.7678 40.5991) (width 0.254) (layer F.Cu) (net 2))
 (segment (start 53.34 25.4) (end 52.1461 25.4) (width 0.254) (layer F.Cu) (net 2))
 (segment (start 26.9625 40.5991) (end 27.7678 40.5991) (width 0.254) (layer F.Cu) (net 2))
 (segment (start 41.148 48.1076) (end 35.2763 48.1076) (width 0.254) (layer F.Cu) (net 2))
 (segment (start 35.2763 48.1076) (end 27.7678 40.5991) (width 0.254) (layer F.Cu) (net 2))
 (segment (start 41.3982 48.1076) (end 41.148 48.1076) (width 0.254) (layer F.Cu) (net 2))
 (segment (start 41.3982 48.1076) (end 41.8771 48.1076) (width 0.254) (layer F.Cu) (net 2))
 (segment (start 32.131 32.627) (end 31.4257 32.627) (width 0.254) (layer F.Cu) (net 2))
 (segment (start 31.3836 31.8954) (end 31.4257 31.9375) (width 0.254) (layer F.Cu) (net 2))
 (segment (start 31.4257 31.9375) (end 31.4257 32.627) (width 0.254) (layer F.Cu) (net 2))
 (segment (start 34.7197 32.106) (end 34.5091 31.8954) (width 0.254) (layer F.Cu) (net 2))
 (segment (start 34.5091 31.8954) (end 31.3836 31.8954) (width 0.254) (layer F.Cu) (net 2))
 (segment (start 35.8 32.106) (end 34.7197 32.106) (width 0.254) (layer F.Cu) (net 2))
 (segment (start 58.71 33.75) (end 58.71 34.7303) (width 0.254) (layer F.Cu) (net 2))
 (segment (start 63.21 37.6234) (end 63.4388 37.3946) (width 0.254) (layer F.Cu) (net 2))
 (segment (start 63.4388 37.3946) (end 65.208 37.3946) (width 0.254) (layer F.Cu) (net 2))
 (segment (start 58.71 34.7303) (end 60.3169 34.7303) (width 0.254) (layer F.Cu) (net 2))
 (segment (start 60.3169 34.7303) (end 63.21 37.6234) (width 0.254) (layer F.Cu) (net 2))
 (segment (start 63.21 37.6234) (end 63.21 42.45) (width 0.254) (layer F.Cu) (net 2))
 (segment (start 65.208 37.3946) (end 65.2084 37.3946) (width 0.2498) (layer F.Cu) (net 2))
 (segment (start 65.2084 37.3946) (end 65.253 37.35) (width 0.2498) (layer F.Cu) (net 2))
 (segment (start 65.31 37.35) (end 65.253 37.35) (width 0.254) (layer F.Cu) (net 2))
 (segment (start 26.2763 29.337) (end 26.2763 30.0661) (width 0.254) (layer F.Cu) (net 2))
 (segment (start 55.88 50.8) (end 54.6861 50.8) (width 0.254) (layer F.Cu) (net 2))
 (segment (start 45.72 49.52) (end 46.5503 49.52) (width 0.254) (layer F.Cu) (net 2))
 (segment (start 46.5503 49.52) (end 49.2077 52.1774) (width 0.254) (layer F.Cu) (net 2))
 (segment (start 49.2077 52.1774) (end 53.8041 52.1774) (width 0.254) (layer F.Cu) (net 2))
 (segment (start 53.8041 52.1774) (end 54.6861 51.2954) (width 0.254) (layer F.Cu) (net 2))
 (segment (start 54.6861 51.2954) (end 54.6861 50.8) (width 0.254) (layer F.Cu) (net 2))
 (segment (start 41.8771 48.1076) (end 43.2895 49.52) (width 0.254) (layer F.Cu) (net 2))
 (segment (start 43.2895 49.52) (end 45.72 49.52) (width 0.254) (layer F.Cu) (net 2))
 (segment (start 50.8 25.4) (end 44.45 25.4) (width 0.254) (layer F.Cu) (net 3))
 (segment (start 44.45 25.4) (end 40.4 29.45) (width 0.254) (layer F.Cu) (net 3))
 (segment (start 40.4 29.45) (end 40.4 32.106) (width 0.254) (layer F.Cu) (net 3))
 (segment (start 44.704 32.5) (end 40.794 32.5) (width 0.254) (layer F.Cu) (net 3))
 (segment (start 40.794 32.5) (end 40.4 32.106) (width 0.254) (layer F.Cu) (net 3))
 (segment (start 35.56 35.56) (end 39.624 35.56) (width 0.254) (layer F.Cu) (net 3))
 (segment (start 39.624 35.56) (end 40.4 34.784) (width 0.254) (layer F.Cu) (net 3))
 (segment (start 40.4 34.784) (end 40.4 32.106) (width 0.254) (layer F.Cu) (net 3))
 (segment (start 26.4875 36.7991) (end 26.9625 36.7991) (width 0.254) (layer F.Cu) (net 7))
 (segment (start 33.45 35.56) (end 29.931 35.56) (width 0.254) (layer F.Cu) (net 7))
 (segment (start 29.931 35.56) (end 28.6919 36.7991) (width 0.254) (layer F.Cu) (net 7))
 (segment (start 28.6919 36.7991) (end 26.9625 36.7991) (width 0.254) (layer F.Cu) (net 7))
 (segment (start 56.61 39.85) (end 49.685 39.85) (width 0.254) (layer F.Cu) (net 18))
 (segment (start 49.685 39.85) (end 49.53 40.005) (width 0.254) (layer F.Cu) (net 18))
 (segment (start 58.42 50.8) (end 58.42 48.895) (width 0.254) (layer B.Cu) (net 18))
 (segment (start 58.42 48.895) (end 49.53 40.005) (width 0.254) (layer B.Cu) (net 18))
 (via (at 49.53 40.005) (size 0.8) (layers F.Cu B.Cu) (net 18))
 (segment (start 58.204 43.177) (end 58.21 43.171) (width 0.254) (layer F.Cu) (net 19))
 (segment (start 58.21 43.171) (end 58.21 42.45) (width 0.254) (layer F.Cu) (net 19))
 (segment (start 58.204 43.177) (end 58.204 42.45) (width 0.254) (layer F.Cu) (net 19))
 (segment (start 53.34 50.8) (end 53.34 48.768) (width 0.254) (layer F.Cu) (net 19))
 (segment (start 53.34 48.768) (end 58.204 43.904) (width 0.254) (layer F.Cu) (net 19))
 (segment (start 58.204 43.904) (end 58.204 43.177) (width 0.254) (layer F.Cu) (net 19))
 (segment (start 56.61 39.35) (end 55.635 39.35) (width 0.2032) (layer F.Cu) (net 5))
 (segment (start 55.635 39.35) (end 55.6136 39.3286) (width 0.2032) (layer F.Cu) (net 5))
 (segment (start 55.6136 39.3286) (end 51.7053 39.3286) (width 0.2032) (layer F.Cu) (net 5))
 (segment (start 51.7053 39.3286) (end 50.3794 38.0027) (width 0.2032) (layer F.Cu) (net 5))
 (segment (start 50.3794 38.0027) (end 28.0714 38.0027) (width 0.2032) (layer F.Cu) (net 5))
 (segment (start 28.0714 38.0027) (end 27.975 38.0991) (width 0.2032) (layer F.Cu) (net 5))
 (segment (start 27.975 38.0991) (end 26.9625 38.0991) (width 0.2032) (layer F.Cu) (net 5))
 (segment (start 56.61 38.85) (end 55.635 38.85) (width 0.2032) (layer F.Cu) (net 6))
 (segment (start 55.635 38.85) (end 55.6136 38.8714) (width 0.2032) (layer F.Cu) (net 6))
 (segment (start 55.6136 38.8714) (end 51.8947 38.8714) (width 0.2032) (layer F.Cu) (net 6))
 (segment (start 51.8947 38.8714) (end 50.5688 37.5455) (width 0.2032) (layer F.Cu) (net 6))
 (segment (start 50.5688 37.5455) (end 28.0714 37.5455) (width 0.2032) (layer F.Cu) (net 6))
 (segment (start 28.0714 37.5455) (end 27.975 37.4491) (width 0.2032) (layer F.Cu) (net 6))
 (segment (start 27.975 37.4491) (end 26.9625 37.4491) (width 0.2032) (layer F.Cu) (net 6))
 (segment (start 68.58 49.784) (end 68.58 50.8) (width 0.254) (layer F.Cu) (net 14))
 (segment (start 68.58 49.784) (end 68.58 50.8) (width 0.254) (layer F.Cu) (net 14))
 (segment (start 62.71 42.45) (end 62.71 44.93) (width 0.254) (layer F.Cu) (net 14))
 (segment (start 62.71 44.93) (end 66.548 48.768) (width 0.254) (layer F.Cu) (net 14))
 (segment (start 66.548 48.768) (end 68.072 48.768) (width 0.254) (layer F.Cu) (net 14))
 (segment (start 68.072 48.768) (end 68.58 49.276) (width 0.254) (layer F.Cu) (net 14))
 (segment (start 68.58 49.276) (end 68.58 49.784) (width 0.254) (layer F.Cu) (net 14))
 (segment (start 62.21 42.45) (end 62.21 45.192) (width 0.254) (layer F.Cu) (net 15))
 (segment (start 62.21 45.192) (end 66.04 49.022) (width 0.254) (layer F.Cu) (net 15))
 (segment (start 66.04 49.022) (end 66.04 50.8) (width 0.254) (layer F.Cu) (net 15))
 (segment (start 61.21 42.45) (end 61.21 45.208) (width 0.254) (layer F.Cu) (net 16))
 (segment (start 61.21 45.208) (end 63.5 47.498) (width 0.254) (layer F.Cu) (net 16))
 (segment (start 63.5 47.498) (end 63.5 50.8) (width 0.254) (layer F.Cu) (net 16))
 (segment (start 60.96 50.8) (end 60.96 45.974) (width 0.254) (layer F.Cu) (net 17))
 (segment (start 60.96 45.974) (end 60.706 45.72) (width 0.254) (layer F.Cu) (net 17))
 (segment (start 60.706 45.72) (end 60.706 42.454) (width 0.254) (layer F.Cu) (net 17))
 (segment (start 60.706 42.454) (end 60.71 42.45) (width 0.254) (layer F.Cu) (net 17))
 (segment (start 61.71 33.75) (end 61.71 30.468) (width 0.254) (layer F.Cu) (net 9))
 (segment (start 61.71 30.468) (end 58.42 27.178) (width 0.254) (layer F.Cu) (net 9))
 (segment (start 58.42 27.178) (end 58.42 25.4) (width 0.254) (layer F.Cu) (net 9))
 (segment (start 62.21 33.75) (end 62.21 28.936) (width 0.254) (layer F.Cu) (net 10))
 (segment (start 62.21 28.936) (end 60.96 27.686) (width 0.254) (layer F.Cu) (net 10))
 (segment (start 60.96 27.686) (end 60.96 25.4) (width 0.254) (layer F.Cu) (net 10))
 (segment (start 62.71 33.75) (end 62.71 28.984) (width 0.254) (layer F.Cu) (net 11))
 (segment (start 62.71 28.984) (end 63.5 28.194) (width 0.254) (layer F.Cu) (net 11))
 (segment (start 63.5 28.194) (end 63.5 25.4) (width 0.254) (layer F.Cu) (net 11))
 (segment (start 63.21 33.75) (end 63.21 33.564) (width 0.254) (layer F.Cu) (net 12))
 (segment (start 63.21 33.564) (end 63.2528 33.5212) (width 0.254) (layer F.Cu) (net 12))
 (segment (start 63.2528 33.5212) (end 63.2528 30.4732) (width 0.254) (layer F.Cu) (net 12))
 (segment (start 63.2528 30.4732) (end 66.04 27.686) (width 0.254) (layer F.Cu) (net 12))
 (segment (start 66.04 27.686) (end 66.04 25.4) (width 0.254) (layer F.Cu) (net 12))
 (segment (start 68.58 25.4) (end 68.58 26.162) (width 0.254) (layer F.Cu) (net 13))
 (segment (start 68.58 26.162) (end 63.71 31.032) (width 0.254) (layer F.Cu) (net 13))
 (segment (start 63.71 31.032) (end 63.71 33.75) (width 0.254) (layer F.Cu) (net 13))
 (segment (start 61.21 33.75) (end 61.21 30.984) (width 0.254) (layer F.Cu) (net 8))
 (segment (start 61.21 30.984) (end 55.88 25.654) (width 0.254) (layer F.Cu) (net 8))
 (segment (start 55.88 25.654) (end 55.88 25.4) (width 0.254) (layer F.Cu) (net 8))
 (segment (start 24.777 31.115) (end 24.777 29.3377) (width 0.254) (layer F.Cu) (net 45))
 (segment (start 24.777 29.3377) (end 24.7777 29.337) (width 0.254) (layer F.Cu) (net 45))
 (segment (start 41.148 46.609) (end 41.148 44.958) (width 0.254) (layer F.Cu) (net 46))
 (segment (start 41.148 43.458) (end 41.148 39.878) (width 0.254) (layer F.Cu) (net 31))
 (segment (start 41.148 39.878) (end 41.402 39.624) (width 0.254) (layer F.Cu) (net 31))
 (segment (start 56.61 35.35) (end 51.606 35.35) (width 0.254) (layer F.Cu) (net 31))
 (segment (start 51.606 35.35) (end 51.562 35.306) (width 0.254) (layer F.Cu) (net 31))
 (segment (start 41.402 39.624) (end 45.72 35.306) (width 0.254) (layer B.Cu) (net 31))
 (segment (start 45.72 35.306) (end 51.562 35.306) (width 0.254) (layer B.Cu) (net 31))
 (via (at 41.402 39.624) (size 0.8) (layers F.Cu B.Cu) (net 31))
 (via (at 51.562 35.306) (size 0.8) (layers F.Cu B.Cu) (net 31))
 (segment (start 45.72 41.92) (end 45.72 40.259) (width 0.254) (layer F.Cu) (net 30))
 (segment (start 45.72 40.259) (end 46.355 39.624) (width 0.254) (layer F.Cu) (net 30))
 (segment (start 56.61 35.85) (end 53.05 35.85) (width 0.254) (layer F.Cu) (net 30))
 (segment (start 53.05 35.85) (end 52.451 36.449) (width 0.254) (layer F.Cu) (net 30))
 (segment (start 46.355 39.624) (end 49.53 36.449) (width 0.254) (layer B.Cu) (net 30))
 (segment (start 49.53 36.449) (end 52.451 36.449) (width 0.254) (layer B.Cu) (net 30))
 (via (at 46.355 39.624) (size 0.8) (layers F.Cu B.Cu) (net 30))
 (via (at 52.451 36.449) (size 0.8) (layers F.Cu B.Cu) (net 30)))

